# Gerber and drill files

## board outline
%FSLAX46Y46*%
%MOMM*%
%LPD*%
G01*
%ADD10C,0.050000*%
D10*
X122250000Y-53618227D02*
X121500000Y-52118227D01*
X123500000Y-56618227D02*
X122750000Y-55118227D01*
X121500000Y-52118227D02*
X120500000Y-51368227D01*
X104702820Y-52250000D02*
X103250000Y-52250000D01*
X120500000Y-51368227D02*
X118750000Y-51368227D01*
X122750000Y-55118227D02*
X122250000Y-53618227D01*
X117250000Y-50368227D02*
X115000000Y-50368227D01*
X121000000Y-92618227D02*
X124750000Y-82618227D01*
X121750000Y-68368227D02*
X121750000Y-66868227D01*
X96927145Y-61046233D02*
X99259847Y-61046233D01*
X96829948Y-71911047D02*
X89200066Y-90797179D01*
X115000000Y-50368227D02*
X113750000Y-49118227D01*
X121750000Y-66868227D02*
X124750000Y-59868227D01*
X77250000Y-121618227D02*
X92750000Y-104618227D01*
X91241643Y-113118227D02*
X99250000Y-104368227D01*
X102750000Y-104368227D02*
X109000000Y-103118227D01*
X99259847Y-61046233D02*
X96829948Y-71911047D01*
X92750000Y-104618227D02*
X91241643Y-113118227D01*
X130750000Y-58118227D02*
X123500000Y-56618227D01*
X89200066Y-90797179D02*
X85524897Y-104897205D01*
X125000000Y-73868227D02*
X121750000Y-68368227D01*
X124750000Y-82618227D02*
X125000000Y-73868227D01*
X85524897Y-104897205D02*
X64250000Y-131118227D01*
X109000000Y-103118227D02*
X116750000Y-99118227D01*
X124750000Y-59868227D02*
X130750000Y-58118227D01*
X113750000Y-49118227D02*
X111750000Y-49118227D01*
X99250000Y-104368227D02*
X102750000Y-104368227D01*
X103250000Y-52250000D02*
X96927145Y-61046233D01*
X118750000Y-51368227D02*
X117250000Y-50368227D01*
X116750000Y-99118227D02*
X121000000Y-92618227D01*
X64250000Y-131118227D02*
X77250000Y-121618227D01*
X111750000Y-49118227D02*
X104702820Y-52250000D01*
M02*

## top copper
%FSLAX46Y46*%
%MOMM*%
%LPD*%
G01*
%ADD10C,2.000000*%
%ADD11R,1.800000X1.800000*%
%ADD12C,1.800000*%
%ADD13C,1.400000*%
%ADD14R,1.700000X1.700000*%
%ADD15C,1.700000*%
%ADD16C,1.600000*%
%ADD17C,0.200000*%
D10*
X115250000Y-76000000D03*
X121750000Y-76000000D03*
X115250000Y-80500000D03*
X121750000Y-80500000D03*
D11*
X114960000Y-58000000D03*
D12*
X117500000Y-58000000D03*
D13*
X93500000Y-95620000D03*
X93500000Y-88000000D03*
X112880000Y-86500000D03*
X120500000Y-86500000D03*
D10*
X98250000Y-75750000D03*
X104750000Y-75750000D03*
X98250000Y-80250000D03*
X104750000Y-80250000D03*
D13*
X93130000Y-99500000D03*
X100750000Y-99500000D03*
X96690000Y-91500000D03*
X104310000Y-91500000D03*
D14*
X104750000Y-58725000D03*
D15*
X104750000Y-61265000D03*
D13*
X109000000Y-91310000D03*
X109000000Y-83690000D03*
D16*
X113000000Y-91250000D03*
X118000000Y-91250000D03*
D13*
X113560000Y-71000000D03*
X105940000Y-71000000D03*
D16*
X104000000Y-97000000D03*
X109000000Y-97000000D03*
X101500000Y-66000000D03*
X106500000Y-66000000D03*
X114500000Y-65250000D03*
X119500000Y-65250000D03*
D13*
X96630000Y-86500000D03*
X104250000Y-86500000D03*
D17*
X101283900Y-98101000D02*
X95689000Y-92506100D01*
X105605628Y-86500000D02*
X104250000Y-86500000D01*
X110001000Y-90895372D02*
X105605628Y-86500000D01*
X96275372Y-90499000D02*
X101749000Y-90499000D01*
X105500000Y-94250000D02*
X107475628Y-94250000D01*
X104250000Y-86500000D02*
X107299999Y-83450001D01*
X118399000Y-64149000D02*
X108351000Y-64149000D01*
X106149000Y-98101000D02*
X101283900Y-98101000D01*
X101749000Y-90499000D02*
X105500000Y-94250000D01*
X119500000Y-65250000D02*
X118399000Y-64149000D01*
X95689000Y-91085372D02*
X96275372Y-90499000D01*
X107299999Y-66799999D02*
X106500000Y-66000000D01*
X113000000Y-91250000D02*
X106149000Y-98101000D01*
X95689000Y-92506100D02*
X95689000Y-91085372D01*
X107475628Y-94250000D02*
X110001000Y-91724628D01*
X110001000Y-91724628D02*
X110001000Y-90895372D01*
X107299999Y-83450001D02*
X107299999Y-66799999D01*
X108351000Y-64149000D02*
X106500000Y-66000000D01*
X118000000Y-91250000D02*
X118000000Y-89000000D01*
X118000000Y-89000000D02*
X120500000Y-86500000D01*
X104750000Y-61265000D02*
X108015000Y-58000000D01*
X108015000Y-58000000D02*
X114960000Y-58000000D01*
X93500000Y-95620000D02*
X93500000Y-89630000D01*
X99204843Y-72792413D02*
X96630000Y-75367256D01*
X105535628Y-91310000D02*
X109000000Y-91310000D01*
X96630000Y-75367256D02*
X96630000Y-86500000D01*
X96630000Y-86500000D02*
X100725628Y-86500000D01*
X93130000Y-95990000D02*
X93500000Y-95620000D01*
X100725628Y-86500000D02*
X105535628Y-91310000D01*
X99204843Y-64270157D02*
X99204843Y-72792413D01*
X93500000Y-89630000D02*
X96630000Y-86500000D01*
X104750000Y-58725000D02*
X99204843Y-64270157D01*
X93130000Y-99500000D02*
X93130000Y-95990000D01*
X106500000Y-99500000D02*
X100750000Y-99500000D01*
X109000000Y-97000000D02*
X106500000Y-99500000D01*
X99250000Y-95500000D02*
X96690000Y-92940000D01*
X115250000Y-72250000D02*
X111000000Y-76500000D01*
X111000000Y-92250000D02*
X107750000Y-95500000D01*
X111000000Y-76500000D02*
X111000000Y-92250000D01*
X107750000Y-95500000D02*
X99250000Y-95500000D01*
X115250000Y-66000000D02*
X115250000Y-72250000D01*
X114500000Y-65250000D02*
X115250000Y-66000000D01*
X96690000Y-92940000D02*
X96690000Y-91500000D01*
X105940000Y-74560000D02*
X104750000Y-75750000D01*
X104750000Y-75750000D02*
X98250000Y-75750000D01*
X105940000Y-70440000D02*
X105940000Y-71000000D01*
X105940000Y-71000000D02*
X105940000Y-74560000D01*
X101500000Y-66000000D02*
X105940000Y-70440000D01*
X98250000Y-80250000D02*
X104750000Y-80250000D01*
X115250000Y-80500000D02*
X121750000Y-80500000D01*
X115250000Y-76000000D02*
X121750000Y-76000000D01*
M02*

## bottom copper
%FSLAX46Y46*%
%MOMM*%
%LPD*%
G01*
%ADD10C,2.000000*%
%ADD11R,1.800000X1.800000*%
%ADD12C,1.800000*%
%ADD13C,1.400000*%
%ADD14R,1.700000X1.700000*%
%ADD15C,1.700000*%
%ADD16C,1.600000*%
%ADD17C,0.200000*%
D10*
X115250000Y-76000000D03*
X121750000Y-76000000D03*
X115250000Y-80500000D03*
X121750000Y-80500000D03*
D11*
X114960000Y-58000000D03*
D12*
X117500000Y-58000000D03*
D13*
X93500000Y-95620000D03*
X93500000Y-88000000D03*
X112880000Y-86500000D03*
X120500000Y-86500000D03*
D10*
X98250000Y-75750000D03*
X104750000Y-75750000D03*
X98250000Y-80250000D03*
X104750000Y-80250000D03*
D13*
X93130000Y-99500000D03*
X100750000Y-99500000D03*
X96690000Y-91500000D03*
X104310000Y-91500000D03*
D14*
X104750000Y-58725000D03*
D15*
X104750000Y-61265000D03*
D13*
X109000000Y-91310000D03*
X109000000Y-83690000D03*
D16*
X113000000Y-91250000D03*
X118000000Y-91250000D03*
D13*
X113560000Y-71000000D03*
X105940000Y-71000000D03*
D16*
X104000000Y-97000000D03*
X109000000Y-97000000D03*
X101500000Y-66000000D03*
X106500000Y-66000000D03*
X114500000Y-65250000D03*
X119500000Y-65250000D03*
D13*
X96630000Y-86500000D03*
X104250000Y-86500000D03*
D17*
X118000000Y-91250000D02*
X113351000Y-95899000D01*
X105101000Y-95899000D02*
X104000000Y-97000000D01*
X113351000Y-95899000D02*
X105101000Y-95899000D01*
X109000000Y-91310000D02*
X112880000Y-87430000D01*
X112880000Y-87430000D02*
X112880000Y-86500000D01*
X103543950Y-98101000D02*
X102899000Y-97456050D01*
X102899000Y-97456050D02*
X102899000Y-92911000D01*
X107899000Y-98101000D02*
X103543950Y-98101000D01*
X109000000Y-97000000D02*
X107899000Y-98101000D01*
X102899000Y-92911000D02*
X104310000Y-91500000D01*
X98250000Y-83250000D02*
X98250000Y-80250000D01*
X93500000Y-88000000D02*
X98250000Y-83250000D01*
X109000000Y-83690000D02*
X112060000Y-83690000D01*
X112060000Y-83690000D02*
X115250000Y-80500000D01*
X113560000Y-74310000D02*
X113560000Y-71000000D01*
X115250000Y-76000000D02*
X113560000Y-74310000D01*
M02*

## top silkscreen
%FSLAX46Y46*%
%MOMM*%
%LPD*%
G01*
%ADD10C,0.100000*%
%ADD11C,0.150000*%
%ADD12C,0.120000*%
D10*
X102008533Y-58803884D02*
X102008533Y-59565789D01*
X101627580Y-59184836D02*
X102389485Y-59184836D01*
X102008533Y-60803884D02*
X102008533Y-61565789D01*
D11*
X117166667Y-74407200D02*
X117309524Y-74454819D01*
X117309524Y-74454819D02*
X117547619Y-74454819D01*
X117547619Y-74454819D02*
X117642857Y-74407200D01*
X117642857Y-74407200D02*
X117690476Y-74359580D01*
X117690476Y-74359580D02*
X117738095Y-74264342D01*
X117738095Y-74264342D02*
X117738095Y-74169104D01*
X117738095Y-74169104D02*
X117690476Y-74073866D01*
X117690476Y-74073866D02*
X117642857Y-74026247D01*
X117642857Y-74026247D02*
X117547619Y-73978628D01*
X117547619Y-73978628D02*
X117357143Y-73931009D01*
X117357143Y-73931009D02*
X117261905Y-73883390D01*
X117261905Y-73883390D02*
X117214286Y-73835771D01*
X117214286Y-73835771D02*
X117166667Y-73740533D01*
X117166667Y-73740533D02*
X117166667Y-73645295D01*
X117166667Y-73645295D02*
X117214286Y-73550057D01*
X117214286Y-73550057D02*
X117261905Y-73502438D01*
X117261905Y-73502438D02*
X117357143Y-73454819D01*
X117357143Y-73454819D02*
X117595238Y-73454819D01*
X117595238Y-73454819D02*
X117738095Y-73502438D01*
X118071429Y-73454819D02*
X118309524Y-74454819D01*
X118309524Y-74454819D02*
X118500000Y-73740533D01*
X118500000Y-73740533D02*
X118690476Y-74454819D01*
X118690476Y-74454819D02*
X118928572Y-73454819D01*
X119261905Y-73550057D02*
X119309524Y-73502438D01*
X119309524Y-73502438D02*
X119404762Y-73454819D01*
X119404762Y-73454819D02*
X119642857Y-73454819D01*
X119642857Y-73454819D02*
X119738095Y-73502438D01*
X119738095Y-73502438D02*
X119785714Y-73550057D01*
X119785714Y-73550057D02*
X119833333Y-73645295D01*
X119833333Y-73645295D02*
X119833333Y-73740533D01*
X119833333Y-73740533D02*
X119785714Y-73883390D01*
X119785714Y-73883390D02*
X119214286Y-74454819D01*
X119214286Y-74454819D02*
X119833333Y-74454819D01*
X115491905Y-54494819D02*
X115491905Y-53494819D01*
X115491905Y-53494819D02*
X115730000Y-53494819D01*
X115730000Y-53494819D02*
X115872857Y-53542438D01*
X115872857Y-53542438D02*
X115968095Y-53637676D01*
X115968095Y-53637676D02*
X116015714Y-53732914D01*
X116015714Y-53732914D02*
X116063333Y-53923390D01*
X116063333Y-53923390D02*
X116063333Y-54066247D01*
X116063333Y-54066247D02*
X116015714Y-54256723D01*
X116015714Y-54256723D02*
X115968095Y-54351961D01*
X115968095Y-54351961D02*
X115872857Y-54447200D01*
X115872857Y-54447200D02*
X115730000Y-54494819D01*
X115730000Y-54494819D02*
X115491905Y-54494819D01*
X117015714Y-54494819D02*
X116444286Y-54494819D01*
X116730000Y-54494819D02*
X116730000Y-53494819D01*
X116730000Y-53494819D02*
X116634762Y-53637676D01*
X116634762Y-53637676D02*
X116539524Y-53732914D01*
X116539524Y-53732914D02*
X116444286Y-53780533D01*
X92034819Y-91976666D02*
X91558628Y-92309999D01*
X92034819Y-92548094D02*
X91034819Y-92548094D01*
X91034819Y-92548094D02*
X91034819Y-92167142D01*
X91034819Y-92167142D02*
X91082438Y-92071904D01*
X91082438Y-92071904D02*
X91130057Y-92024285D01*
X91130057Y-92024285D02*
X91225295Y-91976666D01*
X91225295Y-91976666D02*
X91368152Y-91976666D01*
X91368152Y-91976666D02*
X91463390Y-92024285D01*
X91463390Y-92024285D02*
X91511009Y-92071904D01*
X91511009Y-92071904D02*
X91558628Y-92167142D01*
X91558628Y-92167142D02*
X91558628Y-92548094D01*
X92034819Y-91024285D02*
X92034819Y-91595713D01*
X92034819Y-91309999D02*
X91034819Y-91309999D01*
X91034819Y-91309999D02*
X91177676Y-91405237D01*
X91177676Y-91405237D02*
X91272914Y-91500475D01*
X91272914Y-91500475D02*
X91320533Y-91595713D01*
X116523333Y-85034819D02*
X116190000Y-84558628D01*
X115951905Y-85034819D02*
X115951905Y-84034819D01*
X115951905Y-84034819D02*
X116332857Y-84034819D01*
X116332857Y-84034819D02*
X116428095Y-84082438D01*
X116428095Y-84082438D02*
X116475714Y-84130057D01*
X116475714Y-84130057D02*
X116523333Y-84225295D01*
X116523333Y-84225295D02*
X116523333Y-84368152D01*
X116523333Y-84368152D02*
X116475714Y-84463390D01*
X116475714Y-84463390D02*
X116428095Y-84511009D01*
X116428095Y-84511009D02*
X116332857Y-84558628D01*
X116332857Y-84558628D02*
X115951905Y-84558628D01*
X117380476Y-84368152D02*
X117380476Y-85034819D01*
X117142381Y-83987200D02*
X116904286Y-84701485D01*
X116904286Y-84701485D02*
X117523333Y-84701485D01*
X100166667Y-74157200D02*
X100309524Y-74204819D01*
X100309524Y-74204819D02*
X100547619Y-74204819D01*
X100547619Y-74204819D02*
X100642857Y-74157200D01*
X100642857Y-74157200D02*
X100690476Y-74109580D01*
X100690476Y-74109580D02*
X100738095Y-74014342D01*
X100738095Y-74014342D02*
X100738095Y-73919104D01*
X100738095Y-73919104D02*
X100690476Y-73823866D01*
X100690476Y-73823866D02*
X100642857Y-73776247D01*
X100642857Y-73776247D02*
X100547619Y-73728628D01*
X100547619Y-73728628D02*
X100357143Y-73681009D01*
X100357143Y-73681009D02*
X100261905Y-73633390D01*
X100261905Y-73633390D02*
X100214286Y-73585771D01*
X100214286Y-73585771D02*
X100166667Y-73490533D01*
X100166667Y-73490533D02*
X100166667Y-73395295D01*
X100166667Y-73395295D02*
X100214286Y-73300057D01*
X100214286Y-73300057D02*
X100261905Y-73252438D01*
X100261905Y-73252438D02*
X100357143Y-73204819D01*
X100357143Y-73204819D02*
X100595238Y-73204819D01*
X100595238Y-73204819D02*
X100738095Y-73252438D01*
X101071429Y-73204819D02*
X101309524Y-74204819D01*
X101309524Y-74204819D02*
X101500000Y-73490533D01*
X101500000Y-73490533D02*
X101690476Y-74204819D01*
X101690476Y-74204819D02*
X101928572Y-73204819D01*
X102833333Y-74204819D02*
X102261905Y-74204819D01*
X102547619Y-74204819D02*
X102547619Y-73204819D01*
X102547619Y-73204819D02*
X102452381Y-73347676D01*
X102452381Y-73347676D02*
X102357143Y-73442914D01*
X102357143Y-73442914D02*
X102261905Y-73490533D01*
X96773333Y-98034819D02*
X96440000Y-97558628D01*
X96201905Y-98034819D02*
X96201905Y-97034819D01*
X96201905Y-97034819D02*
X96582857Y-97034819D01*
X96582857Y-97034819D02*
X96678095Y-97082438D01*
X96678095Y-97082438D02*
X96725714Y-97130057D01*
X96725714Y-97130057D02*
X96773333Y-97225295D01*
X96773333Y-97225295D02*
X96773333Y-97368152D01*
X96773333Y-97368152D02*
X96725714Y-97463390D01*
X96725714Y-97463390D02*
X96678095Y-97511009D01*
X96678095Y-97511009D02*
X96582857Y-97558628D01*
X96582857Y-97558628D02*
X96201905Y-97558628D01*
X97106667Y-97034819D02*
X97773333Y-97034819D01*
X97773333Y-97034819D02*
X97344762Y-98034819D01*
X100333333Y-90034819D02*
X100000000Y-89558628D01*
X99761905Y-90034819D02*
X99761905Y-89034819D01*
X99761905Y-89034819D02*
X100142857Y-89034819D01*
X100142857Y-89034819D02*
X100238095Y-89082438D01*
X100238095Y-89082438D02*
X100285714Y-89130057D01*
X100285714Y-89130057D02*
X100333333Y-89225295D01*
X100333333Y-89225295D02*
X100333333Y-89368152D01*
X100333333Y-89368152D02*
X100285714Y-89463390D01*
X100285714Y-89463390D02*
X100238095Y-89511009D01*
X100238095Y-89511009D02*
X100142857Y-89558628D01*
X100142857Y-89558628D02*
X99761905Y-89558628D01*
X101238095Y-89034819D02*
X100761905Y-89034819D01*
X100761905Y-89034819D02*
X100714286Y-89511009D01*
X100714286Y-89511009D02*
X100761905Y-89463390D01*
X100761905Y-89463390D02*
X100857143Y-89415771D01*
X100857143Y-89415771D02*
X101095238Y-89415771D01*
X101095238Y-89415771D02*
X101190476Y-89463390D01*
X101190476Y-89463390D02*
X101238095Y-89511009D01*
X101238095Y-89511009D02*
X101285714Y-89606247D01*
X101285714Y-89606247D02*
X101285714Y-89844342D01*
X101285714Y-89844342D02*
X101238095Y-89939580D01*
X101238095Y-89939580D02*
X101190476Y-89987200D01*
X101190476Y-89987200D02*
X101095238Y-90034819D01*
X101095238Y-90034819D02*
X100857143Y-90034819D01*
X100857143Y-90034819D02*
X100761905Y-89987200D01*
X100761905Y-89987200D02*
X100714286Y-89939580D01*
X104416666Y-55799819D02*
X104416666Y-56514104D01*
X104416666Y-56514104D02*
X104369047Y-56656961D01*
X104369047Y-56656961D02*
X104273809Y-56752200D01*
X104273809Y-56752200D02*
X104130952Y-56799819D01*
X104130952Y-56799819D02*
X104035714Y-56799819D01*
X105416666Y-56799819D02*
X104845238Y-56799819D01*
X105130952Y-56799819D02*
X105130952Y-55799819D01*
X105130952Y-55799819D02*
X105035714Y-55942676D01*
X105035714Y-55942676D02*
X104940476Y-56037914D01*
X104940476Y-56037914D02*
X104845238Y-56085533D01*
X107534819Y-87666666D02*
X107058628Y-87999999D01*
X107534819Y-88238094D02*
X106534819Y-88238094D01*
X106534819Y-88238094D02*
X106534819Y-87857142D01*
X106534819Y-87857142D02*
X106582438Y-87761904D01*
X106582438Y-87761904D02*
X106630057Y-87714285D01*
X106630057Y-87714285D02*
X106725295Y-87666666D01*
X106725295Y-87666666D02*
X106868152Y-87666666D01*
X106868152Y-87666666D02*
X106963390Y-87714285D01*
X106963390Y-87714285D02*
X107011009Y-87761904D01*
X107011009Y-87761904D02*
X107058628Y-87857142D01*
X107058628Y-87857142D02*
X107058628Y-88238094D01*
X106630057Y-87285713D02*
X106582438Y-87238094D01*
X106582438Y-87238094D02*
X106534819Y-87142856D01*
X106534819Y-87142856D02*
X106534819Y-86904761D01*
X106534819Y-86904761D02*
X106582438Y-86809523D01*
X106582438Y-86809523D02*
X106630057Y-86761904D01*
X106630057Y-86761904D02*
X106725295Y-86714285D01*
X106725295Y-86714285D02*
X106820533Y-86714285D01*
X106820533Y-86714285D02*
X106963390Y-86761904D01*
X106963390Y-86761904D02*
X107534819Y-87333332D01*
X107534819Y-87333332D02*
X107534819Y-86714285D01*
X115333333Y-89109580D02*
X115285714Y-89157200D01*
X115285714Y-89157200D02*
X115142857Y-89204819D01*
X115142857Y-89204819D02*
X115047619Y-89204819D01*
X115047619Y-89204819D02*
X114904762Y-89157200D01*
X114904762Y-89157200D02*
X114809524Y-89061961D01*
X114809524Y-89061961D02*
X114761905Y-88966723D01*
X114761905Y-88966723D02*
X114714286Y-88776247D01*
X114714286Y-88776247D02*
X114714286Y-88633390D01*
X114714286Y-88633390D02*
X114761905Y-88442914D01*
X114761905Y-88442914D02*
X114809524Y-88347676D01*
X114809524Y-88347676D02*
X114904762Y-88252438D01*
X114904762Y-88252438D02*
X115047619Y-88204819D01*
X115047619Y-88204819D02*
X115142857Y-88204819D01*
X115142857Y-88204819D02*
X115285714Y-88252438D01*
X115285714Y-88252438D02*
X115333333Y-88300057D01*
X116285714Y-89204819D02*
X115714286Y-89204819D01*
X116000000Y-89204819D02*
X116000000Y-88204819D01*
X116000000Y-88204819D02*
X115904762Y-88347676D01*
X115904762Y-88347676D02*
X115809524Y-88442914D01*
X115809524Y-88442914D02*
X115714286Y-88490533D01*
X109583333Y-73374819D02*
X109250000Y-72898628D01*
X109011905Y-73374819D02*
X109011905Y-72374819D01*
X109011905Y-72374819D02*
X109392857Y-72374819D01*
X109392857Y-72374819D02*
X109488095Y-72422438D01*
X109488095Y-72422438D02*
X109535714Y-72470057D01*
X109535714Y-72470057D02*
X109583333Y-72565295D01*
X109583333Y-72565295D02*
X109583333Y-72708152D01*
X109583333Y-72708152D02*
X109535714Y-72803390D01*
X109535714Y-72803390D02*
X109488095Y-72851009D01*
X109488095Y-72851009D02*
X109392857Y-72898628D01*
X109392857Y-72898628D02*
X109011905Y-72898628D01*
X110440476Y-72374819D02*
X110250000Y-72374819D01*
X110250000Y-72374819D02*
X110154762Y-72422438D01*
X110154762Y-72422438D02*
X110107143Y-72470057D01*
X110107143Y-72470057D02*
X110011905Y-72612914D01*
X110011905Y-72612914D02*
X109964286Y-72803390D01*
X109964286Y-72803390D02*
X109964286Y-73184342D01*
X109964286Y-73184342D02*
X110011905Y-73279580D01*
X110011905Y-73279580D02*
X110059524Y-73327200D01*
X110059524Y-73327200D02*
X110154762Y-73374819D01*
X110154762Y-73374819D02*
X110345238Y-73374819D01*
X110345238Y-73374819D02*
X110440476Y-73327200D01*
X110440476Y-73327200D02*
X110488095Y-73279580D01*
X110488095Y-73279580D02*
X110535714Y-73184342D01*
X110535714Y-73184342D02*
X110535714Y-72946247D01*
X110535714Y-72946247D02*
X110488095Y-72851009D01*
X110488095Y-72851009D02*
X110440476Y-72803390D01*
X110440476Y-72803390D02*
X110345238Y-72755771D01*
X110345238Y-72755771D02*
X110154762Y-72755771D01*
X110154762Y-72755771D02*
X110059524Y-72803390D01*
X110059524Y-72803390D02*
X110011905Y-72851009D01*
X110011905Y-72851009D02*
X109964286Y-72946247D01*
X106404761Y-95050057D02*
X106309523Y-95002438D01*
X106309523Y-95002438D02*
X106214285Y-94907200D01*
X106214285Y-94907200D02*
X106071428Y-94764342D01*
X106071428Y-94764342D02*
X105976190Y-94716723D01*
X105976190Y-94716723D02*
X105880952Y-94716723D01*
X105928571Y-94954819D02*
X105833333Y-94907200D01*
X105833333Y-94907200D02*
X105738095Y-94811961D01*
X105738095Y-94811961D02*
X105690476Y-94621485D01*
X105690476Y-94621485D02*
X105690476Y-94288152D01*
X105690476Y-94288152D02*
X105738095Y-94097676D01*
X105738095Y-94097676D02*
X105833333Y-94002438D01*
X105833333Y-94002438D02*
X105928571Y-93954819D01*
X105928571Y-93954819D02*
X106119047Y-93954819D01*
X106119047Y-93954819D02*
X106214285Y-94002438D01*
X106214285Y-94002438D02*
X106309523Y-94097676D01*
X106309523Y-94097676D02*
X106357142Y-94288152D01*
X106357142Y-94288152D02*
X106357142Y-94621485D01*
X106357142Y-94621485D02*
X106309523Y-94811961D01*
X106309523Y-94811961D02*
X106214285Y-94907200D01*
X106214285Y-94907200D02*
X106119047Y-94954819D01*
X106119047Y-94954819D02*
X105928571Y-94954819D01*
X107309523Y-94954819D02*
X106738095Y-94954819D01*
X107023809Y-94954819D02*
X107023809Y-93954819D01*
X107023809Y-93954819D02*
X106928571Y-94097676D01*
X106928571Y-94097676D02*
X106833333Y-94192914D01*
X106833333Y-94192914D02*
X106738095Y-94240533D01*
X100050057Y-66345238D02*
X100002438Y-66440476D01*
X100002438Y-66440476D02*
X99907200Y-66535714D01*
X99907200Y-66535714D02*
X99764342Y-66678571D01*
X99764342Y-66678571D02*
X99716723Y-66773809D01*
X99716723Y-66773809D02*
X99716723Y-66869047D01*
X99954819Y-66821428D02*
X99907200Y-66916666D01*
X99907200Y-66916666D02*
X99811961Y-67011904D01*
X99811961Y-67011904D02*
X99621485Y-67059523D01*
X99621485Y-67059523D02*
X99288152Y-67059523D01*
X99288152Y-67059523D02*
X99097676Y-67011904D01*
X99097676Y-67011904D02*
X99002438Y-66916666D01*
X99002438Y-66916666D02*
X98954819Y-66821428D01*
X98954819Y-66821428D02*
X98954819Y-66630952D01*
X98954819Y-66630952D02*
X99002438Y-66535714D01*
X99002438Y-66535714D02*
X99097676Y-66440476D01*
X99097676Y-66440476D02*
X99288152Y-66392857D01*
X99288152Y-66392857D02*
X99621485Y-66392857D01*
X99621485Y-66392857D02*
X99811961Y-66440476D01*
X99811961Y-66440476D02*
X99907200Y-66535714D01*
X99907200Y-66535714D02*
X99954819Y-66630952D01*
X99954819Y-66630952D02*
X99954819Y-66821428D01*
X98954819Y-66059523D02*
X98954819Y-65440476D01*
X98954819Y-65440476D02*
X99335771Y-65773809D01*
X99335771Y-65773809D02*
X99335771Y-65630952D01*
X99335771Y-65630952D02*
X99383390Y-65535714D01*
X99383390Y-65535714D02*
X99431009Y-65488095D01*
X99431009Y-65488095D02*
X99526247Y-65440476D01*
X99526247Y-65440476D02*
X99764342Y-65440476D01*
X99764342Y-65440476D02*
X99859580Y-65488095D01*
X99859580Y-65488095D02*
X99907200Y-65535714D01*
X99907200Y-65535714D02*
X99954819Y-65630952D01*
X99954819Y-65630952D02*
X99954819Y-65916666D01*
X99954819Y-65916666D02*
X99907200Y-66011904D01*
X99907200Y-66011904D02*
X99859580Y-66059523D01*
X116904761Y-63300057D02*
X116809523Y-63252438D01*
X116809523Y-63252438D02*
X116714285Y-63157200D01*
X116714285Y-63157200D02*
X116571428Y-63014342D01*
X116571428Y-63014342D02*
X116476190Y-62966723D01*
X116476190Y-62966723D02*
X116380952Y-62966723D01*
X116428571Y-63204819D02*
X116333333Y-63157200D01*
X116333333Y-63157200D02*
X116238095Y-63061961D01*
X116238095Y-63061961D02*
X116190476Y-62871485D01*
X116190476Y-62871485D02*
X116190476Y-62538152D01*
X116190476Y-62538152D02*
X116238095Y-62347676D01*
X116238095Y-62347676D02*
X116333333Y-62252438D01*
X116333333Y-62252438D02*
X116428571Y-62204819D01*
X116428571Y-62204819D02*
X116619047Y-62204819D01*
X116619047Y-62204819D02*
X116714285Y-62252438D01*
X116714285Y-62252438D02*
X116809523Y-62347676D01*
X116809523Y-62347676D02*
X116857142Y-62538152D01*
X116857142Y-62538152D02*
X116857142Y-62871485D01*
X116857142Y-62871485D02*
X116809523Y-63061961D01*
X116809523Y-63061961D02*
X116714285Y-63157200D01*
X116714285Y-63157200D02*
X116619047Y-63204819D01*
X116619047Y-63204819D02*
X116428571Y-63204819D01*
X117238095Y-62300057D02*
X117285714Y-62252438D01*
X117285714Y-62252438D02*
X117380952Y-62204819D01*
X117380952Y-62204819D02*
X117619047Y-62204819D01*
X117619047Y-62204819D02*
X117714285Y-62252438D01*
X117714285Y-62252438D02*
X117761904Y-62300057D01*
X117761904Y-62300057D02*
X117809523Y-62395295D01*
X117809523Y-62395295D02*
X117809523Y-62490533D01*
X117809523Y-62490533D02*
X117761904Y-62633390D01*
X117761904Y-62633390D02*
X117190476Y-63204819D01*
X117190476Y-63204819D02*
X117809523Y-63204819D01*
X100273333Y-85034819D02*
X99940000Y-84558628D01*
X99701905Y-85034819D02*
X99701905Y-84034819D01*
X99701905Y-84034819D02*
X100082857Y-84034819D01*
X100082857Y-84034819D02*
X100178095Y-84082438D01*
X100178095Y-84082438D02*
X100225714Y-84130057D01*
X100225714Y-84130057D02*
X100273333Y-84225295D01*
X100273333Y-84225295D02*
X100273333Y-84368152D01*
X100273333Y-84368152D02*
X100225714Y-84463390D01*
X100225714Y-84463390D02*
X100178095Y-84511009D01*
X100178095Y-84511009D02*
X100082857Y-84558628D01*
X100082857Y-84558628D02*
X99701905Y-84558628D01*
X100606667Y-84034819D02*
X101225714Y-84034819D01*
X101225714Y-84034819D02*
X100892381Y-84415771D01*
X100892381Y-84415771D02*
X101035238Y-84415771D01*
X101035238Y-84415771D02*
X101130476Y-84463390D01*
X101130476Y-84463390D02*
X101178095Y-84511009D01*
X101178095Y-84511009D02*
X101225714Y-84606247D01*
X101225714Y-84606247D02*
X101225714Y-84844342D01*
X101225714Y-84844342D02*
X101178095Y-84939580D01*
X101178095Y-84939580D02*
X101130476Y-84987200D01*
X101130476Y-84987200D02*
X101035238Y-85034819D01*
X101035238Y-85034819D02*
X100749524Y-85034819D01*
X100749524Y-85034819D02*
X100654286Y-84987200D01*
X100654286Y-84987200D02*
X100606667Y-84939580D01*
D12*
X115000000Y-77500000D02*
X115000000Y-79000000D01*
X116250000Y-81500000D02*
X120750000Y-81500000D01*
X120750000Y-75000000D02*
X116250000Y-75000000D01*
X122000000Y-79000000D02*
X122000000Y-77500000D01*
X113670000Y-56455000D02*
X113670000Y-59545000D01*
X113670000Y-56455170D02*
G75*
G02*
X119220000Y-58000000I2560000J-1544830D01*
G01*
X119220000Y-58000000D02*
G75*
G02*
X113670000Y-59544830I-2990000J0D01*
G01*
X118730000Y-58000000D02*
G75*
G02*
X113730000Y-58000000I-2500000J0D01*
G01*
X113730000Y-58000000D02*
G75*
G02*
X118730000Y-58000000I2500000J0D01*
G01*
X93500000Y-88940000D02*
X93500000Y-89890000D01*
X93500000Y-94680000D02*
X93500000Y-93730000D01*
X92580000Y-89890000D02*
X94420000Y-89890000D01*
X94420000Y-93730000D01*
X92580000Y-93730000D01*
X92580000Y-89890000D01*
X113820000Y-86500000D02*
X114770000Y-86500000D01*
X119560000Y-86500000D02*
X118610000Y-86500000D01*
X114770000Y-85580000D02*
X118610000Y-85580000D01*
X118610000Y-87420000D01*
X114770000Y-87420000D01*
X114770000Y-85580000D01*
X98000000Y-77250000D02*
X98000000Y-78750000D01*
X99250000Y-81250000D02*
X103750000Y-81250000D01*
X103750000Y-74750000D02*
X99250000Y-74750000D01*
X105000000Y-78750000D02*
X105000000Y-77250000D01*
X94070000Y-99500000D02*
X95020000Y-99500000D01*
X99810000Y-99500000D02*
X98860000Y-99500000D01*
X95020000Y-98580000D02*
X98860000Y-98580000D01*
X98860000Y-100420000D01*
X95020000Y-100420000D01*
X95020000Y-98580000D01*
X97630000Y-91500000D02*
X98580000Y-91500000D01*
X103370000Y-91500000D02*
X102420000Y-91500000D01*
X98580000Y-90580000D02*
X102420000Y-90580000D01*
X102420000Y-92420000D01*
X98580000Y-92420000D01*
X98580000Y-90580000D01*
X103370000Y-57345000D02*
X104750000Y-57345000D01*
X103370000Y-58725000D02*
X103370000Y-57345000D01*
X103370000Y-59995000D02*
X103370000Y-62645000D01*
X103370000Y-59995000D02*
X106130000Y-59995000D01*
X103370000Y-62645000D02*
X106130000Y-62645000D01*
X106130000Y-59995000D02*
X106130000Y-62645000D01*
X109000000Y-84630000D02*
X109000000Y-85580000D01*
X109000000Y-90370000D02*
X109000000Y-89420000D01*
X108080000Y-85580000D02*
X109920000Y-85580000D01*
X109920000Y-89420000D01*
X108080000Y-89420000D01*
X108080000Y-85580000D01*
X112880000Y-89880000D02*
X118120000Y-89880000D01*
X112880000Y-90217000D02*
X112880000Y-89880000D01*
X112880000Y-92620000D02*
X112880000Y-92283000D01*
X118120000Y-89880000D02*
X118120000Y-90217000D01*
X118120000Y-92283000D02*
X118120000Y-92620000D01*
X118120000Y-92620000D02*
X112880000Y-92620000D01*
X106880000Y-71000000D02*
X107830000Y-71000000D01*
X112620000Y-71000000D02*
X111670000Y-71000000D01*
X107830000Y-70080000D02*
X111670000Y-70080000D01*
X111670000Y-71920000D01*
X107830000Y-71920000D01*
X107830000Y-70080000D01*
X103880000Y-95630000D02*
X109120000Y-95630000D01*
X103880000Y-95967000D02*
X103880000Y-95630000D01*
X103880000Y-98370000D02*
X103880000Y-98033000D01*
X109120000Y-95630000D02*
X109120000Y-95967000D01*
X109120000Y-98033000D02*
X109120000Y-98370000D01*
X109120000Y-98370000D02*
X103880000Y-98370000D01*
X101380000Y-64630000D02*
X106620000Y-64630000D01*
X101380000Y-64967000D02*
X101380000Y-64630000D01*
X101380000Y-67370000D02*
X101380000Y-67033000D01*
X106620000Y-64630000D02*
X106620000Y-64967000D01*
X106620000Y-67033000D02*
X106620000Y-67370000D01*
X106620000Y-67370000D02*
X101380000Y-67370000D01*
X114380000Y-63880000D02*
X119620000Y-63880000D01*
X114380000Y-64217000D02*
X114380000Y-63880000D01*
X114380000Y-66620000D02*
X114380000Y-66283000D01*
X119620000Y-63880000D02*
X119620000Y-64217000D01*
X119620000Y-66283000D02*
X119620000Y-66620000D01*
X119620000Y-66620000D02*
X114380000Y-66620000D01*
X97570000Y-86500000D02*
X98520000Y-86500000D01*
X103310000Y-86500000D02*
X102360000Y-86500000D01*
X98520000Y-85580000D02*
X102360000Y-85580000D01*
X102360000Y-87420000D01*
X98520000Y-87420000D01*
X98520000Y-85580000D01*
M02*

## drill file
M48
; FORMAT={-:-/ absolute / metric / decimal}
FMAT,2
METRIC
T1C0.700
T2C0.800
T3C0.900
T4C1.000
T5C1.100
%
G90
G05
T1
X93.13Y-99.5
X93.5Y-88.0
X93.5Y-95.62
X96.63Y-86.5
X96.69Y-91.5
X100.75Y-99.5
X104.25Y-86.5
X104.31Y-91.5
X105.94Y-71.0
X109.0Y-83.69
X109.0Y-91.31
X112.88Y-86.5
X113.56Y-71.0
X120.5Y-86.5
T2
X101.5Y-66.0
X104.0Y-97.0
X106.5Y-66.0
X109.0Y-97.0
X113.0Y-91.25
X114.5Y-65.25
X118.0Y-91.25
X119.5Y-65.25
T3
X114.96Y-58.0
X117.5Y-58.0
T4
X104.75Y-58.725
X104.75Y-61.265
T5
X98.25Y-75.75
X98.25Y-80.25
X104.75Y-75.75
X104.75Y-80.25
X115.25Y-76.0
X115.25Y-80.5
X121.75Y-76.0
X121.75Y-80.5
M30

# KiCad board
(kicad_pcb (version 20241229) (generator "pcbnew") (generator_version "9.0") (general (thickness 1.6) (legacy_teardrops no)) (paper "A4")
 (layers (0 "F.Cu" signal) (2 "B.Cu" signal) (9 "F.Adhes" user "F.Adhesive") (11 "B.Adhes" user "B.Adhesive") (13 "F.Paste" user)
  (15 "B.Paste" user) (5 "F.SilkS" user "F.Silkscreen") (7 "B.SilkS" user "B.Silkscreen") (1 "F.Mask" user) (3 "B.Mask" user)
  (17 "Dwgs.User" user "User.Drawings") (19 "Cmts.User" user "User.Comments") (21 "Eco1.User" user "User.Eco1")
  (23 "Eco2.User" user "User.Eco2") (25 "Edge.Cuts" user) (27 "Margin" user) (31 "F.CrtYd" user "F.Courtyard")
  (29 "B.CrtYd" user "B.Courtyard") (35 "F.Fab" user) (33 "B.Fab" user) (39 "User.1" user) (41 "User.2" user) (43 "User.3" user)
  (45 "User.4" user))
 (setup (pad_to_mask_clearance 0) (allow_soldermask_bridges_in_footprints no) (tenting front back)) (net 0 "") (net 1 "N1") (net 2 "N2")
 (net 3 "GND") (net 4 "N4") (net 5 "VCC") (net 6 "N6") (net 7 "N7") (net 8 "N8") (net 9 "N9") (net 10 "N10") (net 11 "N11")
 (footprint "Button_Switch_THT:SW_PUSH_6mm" (layer "F.Cu") (at 115.25 76)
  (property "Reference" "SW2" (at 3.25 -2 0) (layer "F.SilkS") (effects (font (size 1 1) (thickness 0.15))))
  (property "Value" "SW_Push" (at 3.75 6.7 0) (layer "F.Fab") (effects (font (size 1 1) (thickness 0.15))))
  (fp_line (start -0.25 1.5) (end -0.25 3) (stroke (width 0.12) (type solid)) (layer "F.SilkS"))
  (fp_line (start 1 5.5) (end 5.5 5.5) (stroke (width 0.12) (type solid)) (layer "F.SilkS"))
  (fp_line (start 5.5 -1) (end 1 -1) (stroke (width 0.12) (type solid)) (layer "F.SilkS"))
  (fp_line (start 6.75 3) (end 6.75 1.5) (stroke (width 0.12) (type solid)) (layer "F.SilkS"))
  (pad "1" thru_hole circle (at 0 0 90) (size 2 2) (drill 1.1) (layers "*.Cu" "*.Mask") (remove_unused_layers no) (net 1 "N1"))
  (pad "1" thru_hole circle (at 6.5 0 90) (size 2 2) (drill 1.1) (layers "*.Cu" "*.Mask") (remove_unused_layers no) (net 1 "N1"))
  (pad "2" thru_hole circle (at 0 4.5 90) (size 2 2) (drill 1.1) (layers "*.Cu" "*.Mask") (remove_unused_layers no) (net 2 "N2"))
  (pad "2" thru_hole circle (at 6.5 4.5 90) (size 2 2) (drill 1.1) (layers "*.Cu" "*.Mask") (remove_unused_layers no) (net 2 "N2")))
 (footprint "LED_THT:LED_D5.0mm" (layer "F.Cu") (at 114.96 58)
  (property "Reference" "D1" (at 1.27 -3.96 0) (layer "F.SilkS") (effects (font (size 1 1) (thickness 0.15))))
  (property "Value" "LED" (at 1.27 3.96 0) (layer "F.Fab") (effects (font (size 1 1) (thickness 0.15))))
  (fp_line (start -1.29 -1.545) (end -1.29 1.545) (stroke (width 0.12) (type solid)) (layer "F.SilkS"))
  (fp_arc (start -1.29 -1.54483) (mid 2.071779 -2.880495) (end 4.26 0) (stroke (width 0.12) (type solid)) (layer "F.SilkS"))
  (fp_arc (start 4.26 0) (mid 2.071779 2.880495) (end -1.29 1.54483) (stroke (width 0.12) (type solid)) (layer "F.SilkS"))
  (fp_circle (center 1.27 0) (end 3.77 0) (stroke (width 0.12) (type solid)) (fill no) (layer "F.SilkS"))
  (pad "1" thru_hole rect (at 0 0) (size 1.8 1.8) (drill 0.9) (layers "*.Cu" "*.Mask") (remove_unused_layers no) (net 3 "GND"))
  (pad "2" thru_hole circle (at 2.54 0) (size 1.8 1.8) (drill 0.9) (layers "*.Cu" "*.Mask") (remove_unused_layers no) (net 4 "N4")))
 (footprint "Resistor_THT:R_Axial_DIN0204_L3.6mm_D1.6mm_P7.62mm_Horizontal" (layer "F.Cu") (at 93.5 95.62 90)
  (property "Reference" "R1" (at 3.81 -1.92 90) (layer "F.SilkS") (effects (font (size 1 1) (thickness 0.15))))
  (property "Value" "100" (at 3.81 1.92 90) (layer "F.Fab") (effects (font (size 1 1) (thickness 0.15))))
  (fp_line (start 6.68 0) (end 5.73 0) (stroke (width 0.12) (type solid)) (layer "F.SilkS"))
  (fp_line (start 0.94 0) (end 1.89 0) (stroke (width 0.12) (type solid)) (layer "F.SilkS"))
  (fp_rect (start 1.89 -0.92) (end 5.73 0.92) (stroke (width 0.12) (type solid)) (fill no) (layer "F.SilkS"))
  (pad "1" thru_hole circle (at 0 0 90) (size 1.4 1.4) (drill 0.7) (layers "*.Cu" "*.Mask") (remove_unused_layers no) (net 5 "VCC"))
  (pad "2" thru_hole circle (at 7.62 0 90) (size 1.4 1.4) (drill 0.7) (layers "*.Cu" "*.Mask") (remove_unused_layers no) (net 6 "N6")))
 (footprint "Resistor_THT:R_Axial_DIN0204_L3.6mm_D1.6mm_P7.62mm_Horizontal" (layer "F.Cu") (at 112.88 86.5)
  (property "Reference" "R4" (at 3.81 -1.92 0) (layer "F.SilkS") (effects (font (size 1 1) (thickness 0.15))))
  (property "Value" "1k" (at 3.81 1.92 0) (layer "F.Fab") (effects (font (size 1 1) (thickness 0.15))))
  (fp_line (start 0.94 0) (end 1.89 0) (stroke (width 0.12) (type solid)) (layer "F.SilkS"))
  (fp_line (start 6.68 0) (end 5.73 0) (stroke (width 0.12) (type solid)) (layer "F.SilkS"))
  (fp_rect (start 1.89 -0.92) (end 5.73 0.92) (stroke (width 0.12) (type solid)) (fill no) (layer "F.SilkS"))
  (pad "1" thru_hole circle (at 0 0) (size 1.4 1.4) (drill 0.7) (layers "*.Cu" "*.Mask") (remove_unused_layers no) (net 5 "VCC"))
  (pad "2" thru_hole circle (at 7.62 0) (size 1.4 1.4) (drill 0.7) (layers "*.Cu" "*.Mask") (remove_unused_layers no) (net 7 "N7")))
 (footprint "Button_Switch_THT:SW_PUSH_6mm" (layer "F.Cu") (at 98.25 75.75)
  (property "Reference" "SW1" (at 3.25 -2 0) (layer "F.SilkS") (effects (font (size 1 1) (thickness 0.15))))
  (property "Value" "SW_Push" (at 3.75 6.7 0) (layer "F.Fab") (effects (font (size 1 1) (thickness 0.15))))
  (fp_line (start -0.25 1.5) (end -0.25 3) (stroke (width 0.12) (type solid)) (layer "F.SilkS"))
  (fp_line (start 1 5.5) (end 5.5 5.5) (stroke (width 0.12) (type solid)) (layer "F.SilkS"))
  (fp_line (start 5.5 -1) (end 1 -1) (stroke (width 0.12) (type solid)) (layer "F.SilkS"))
  (fp_line (start 6.75 3) (end 6.75 1.5) (stroke (width 0.12) (type solid)) (layer "F.SilkS"))
  (pad "1" thru_hole circle (at 0 0 90) (size 2 2) (drill 1.1) (layers "*.Cu" "*.Mask") (remove_unused_layers no) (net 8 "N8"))
  (pad "1" thru_hole circle (at 6.5 0 90) (size 2 2) (drill 1.1) (layers "*.Cu" "*.Mask") (remove_unused_layers no) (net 8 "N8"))
  (pad "2" thru_hole circle (at 0 4.5 90) (size 2 2) (drill 1.1) (layers "*.Cu" "*.Mask") (remove_unused_layers no) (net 6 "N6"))
  (pad "2" thru_hole circle (at 6.5 4.5 90) (size 2 2) (drill 1.1) (layers "*.Cu" "*.Mask") (remove_unused_layers no) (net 6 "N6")))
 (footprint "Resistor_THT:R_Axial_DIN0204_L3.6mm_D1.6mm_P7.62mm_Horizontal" (layer "F.Cu") (at 93.13 99.5)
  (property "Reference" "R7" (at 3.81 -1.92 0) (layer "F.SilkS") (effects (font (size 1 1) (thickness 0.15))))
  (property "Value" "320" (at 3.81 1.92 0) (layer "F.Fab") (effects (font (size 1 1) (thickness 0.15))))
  (fp_line (start 0.94 0) (end 1.89 0) (stroke (width 0.12) (type solid)) (layer "F.SilkS"))
  (fp_line (start 6.68 0) (end 5.73 0) (stroke (width 0.12) (type solid)) (layer "F.SilkS"))
  (fp_rect (start 1.89 -0.92) (end 5.73 0.92) (stroke (width 0.12) (type solid)) (fill no) (layer "F.SilkS"))
  (pad "1" thru_hole circle (at 0 0) (size 1.4 1.4) (drill 0.7) (layers "*.Cu" "*.Mask") (remove_unused_layers no) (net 5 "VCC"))
  (pad "2" thru_hole circle (at 7.62 0) (size 1.4 1.4) (drill 0.7) (layers "*.Cu" "*.Mask") (remove_unused_layers no) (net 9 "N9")))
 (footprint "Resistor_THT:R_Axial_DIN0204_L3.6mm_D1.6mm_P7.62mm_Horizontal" (layer "F.Cu") (at 96.69 91.5)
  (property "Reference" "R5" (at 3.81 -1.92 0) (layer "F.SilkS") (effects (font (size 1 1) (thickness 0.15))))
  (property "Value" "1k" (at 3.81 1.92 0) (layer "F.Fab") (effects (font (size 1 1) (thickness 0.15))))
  (fp_line (start 0.94 0) (end 1.89 0) (stroke (width 0.12) (type solid)) (layer "F.SilkS"))
  (fp_line (start 6.68 0) (end 5.73 0) (stroke (width 0.12) (type solid)) (layer "F.SilkS"))
  (fp_rect (start 1.89 -0.92) (end 5.73 0.92) (stroke (width 0.12) (type solid)) (fill no) (layer "F.SilkS"))
  (pad "1" thru_hole circle (at 0 0) (size 1.4 1.4) (drill 0.7) (layers "*.Cu" "*.Mask") (remove_unused_layers no) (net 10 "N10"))
  (pad "2" thru_hole circle (at 7.62 0) (size 1.4 1.4) (drill 0.7) (layers "*.Cu" "*.Mask") (remove_unused_layers no) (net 9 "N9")))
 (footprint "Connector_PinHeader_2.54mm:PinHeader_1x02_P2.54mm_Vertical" (layer "F.Cu") (at 104.75 58.725)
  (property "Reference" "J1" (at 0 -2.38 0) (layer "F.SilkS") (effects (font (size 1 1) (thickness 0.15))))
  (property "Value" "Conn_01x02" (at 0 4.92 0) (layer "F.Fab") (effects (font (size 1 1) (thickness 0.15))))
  (fp_line (start -1.38 -1.38) (end 0 -1.38) (stroke (width 0.12) (type solid)) (layer "F.SilkS"))
  (fp_line (start -1.38 0) (end -1.38 -1.38) (stroke (width 0.12) (type solid)) (layer "F.SilkS"))
  (fp_line (start -1.38 1.27) (end -1.38 3.92) (stroke (width 0.12) (type solid)) (layer "F.SilkS"))
  (fp_line (start -1.38 1.27) (end 1.38 1.27) (stroke (width 0.12) (type solid)) (layer "F.SilkS"))
  (fp_line (start -1.38 3.92) (end 1.38 3.92) (stroke (width 0.12) (type solid)) (layer "F.SilkS"))
  (fp_line (start 1.38 1.27) (end 1.38 3.92) (stroke (width 0.12) (type solid)) (layer "F.SilkS"))
  (pad "1" thru_hole rect (at 0 0) (size 1.7 1.7) (drill 1) (layers "*.Cu" "*.Mask") (remove_unused_layers no) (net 5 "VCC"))
  (pad "2" thru_hole circle (at 0 2.54) (size 1.7 1.7) (drill 1) (layers "*.Cu" "*.Mask") (remove_unused_layers no) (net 3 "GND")))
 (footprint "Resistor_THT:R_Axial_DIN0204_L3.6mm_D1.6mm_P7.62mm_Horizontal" (layer "F.Cu") (at 109 91.31 90)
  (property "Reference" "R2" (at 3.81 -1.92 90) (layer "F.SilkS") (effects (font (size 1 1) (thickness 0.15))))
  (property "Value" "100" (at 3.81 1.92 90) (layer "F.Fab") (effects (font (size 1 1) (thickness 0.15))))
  (fp_line (start 6.68 0) (end 5.73 0) (stroke (width 0.12) (type solid)) (layer "F.SilkS"))
  (fp_line (start 0.94 0) (end 1.89 0) (stroke (width 0.12) (type solid)) (layer "F.SilkS"))
  (fp_rect (start 1.89 -0.92) (end 5.73 0.92) (stroke (width 0.12) (type solid)) (fill no) (layer "F.SilkS"))
  (pad "1" thru_hole circle (at 0 0 90) (size 1.4 1.4) (drill 0.7) (layers "*.Cu" "*.Mask") (remove_unused_layers no) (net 5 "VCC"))
  (pad "2" thru_hole circle (at 7.62 0 90) (size 1.4 1.4) (drill 0.7) (layers "*.Cu" "*.Mask") (remove_unused_layers no) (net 2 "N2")))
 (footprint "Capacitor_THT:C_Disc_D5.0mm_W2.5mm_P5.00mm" (layer "F.Cu") (at 113 91.25)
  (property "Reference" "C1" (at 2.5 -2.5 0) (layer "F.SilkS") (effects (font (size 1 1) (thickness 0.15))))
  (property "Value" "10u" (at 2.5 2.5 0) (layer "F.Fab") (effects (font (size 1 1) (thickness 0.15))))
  (fp_line (start -0.12 -1.37) (end 5.12 -1.37) (stroke (width 0.12) (type solid)) (layer "F.SilkS"))
  (fp_line (start -0.12 -1.033) (end -0.12 -1.37) (stroke (width 0.12) (type solid)) (layer "F.SilkS"))
  (fp_line (start -0.12 1.37) (end -0.12 1.033) (stroke (width 0.12) (type solid)) (layer "F.SilkS"))
  (fp_line (start 5.12 -1.37) (end 5.12 -1.033) (stroke (width 0.12) (type solid)) (layer "F.SilkS"))
  (fp_line (start 5.12 1.033) (end 5.12 1.37) (stroke (width 0.12) (type solid)) (layer "F.SilkS"))
  (fp_line (start 5.12 1.37) (end -0.12 1.37) (stroke (width 0.12) (type solid)) (layer "F.SilkS"))
  (pad "1" thru_hole circle (at 0 0) (size 1.6 1.6) (drill 0.8) (layers "*.Cu" "*.Mask") (remove_unused_layers no) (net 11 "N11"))
  (pad "2" thru_hole circle (at 5 0) (size 1.6 1.6) (drill 0.8) (layers "*.Cu" "*.Mask") (remove_unused_layers no) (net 7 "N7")))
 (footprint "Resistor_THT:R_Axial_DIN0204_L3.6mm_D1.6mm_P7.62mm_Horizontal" (layer "F.Cu") (at 113.56 71 180)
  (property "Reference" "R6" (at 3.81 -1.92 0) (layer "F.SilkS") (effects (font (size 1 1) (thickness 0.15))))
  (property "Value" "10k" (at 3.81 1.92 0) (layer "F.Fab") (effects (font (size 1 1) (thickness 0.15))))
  (fp_line (start 6.68 0) (end 5.73 0) (stroke (width 0.12) (type solid)) (layer "F.SilkS"))
  (fp_line (start 0.94 0) (end 1.89 0) (stroke (width 0.12) (type solid)) (layer "F.SilkS"))
  (fp_rect (start 1.89 -0.92) (end 5.73 0.92) (stroke (width 0.12) (type solid)) (fill no) (layer "F.SilkS"))
  (pad "1" thru_hole circle (at 0 0 180) (size 1.4 1.4) (drill 0.7) (layers "*.Cu" "*.Mask") (remove_unused_layers no) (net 1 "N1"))
  (pad "2" thru_hole circle (at 7.62 0 180) (size 1.4 1.4) (drill 0.7) (layers "*.Cu" "*.Mask") (remove_unused_layers no) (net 8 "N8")))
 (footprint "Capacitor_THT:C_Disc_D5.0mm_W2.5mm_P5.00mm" (layer "F.Cu") (at 104 97)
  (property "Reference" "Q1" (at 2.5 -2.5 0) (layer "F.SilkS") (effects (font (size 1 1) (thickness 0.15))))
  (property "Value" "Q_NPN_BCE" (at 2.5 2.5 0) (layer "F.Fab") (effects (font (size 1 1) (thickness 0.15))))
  (fp_line (start -0.12 -1.37) (end 5.12 -1.37) (stroke (width 0.12) (type solid)) (layer "F.SilkS"))
  (fp_line (start -0.12 -1.033) (end -0.12 -1.37) (stroke (width 0.12) (type solid)) (layer "F.SilkS"))
  (fp_line (start -0.12 1.37) (end -0.12 1.033) (stroke (width 0.12) (type solid)) (layer "F.SilkS"))
  (fp_line (start 5.12 -1.37) (end 5.12 -1.033) (stroke (width 0.12) (type solid)) (layer "F.SilkS"))
  (fp_line (start 5.12 1.033) (end 5.12 1.37) (stroke (width 0.12) (type solid)) (layer "F.SilkS"))
  (fp_line (start 5.12 1.37) (end -0.12 1.37) (stroke (width 0.12) (type solid)) (layer "F.SilkS"))
  (pad "1" thru_hole circle (at 0 0) (size 1.6 1.6) (drill 0.8) (layers "*.Cu" "*.Mask") (remove_unused_layers no) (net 7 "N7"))
  (pad "2" thru_hole circle (at 5 0) (size 1.6 1.6) (drill 0.8) (layers "*.Cu" "*.Mask") (remove_unused_layers no) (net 9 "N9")))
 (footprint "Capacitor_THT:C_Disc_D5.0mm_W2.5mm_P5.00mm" (layer "F.Cu") (at 101.5 66)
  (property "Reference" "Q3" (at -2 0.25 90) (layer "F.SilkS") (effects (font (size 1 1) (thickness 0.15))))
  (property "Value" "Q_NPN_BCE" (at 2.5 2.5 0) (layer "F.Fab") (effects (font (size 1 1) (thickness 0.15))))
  (fp_line (start -0.12 -1.37) (end 5.12 -1.37) (stroke (width 0.12) (type solid)) (layer "F.SilkS"))
  (fp_line (start -0.12 -1.033) (end -0.12 -1.37) (stroke (width 0.12) (type solid)) (layer "F.SilkS"))
  (fp_line (start -0.12 1.37) (end -0.12 1.033) (stroke (width 0.12) (type solid)) (layer "F.SilkS"))
  (fp_line (start 5.12 -1.37) (end 5.12 -1.033) (stroke (width 0.12) (type solid)) (layer "F.SilkS"))
  (fp_line (start 5.12 1.033) (end 5.12 1.37) (stroke (width 0.12) (type solid)) (layer "F.SilkS"))
  (fp_line (start 5.12 1.37) (end -0.12 1.37) (stroke (width 0.12) (type solid)) (layer "F.SilkS"))
  (pad "1" thru_hole circle (at 0 0) (size 1.6 1.6) (drill 0.8) (layers "*.Cu" "*.Mask") (remove_unused_layers no) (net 8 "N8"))
  (pad "2" thru_hole circle (at 5 0) (size 1.6 1.6) (drill 0.8) (layers "*.Cu" "*.Mask") (remove_unused_layers no) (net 11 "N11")))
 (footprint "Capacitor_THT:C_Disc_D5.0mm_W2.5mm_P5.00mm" (layer "F.Cu") (at 114.5 65.25)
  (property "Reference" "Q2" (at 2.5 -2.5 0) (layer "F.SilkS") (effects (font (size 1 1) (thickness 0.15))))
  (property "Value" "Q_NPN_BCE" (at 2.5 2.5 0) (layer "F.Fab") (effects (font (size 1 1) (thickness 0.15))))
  (fp_line (start -0.12 -1.37) (end 5.12 -1.37) (stroke (width 0.12) (type solid)) (layer "F.SilkS"))
  (fp_line (start -0.12 -1.033) (end -0.12 -1.37) (stroke (width 0.12) (type solid)) (layer "F.SilkS"))
  (fp_line (start -0.12 1.37) (end -0.12 1.033) (stroke (width 0.12) (type solid)) (layer "F.SilkS"))
  (fp_line (start 5.12 -1.37) (end 5.12 -1.033) (stroke (width 0.12) (type solid)) (layer "F.SilkS"))
  (fp_line (start 5.12 1.033) (end 5.12 1.37) (stroke (width 0.12) (type solid)) (layer "F.SilkS"))
  (fp_line (start 5.12 1.37) (end -0.12 1.37) (stroke (width 0.12) (type solid)) (layer "F.SilkS"))
  (pad "1" thru_hole circle (at 0 0) (size 1.6 1.6) (drill 0.8) (layers "*.Cu" "*.Mask") (remove_unused_layers no) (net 10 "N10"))
  (pad "2" thru_hole circle (at 5 0) (size 1.6 1.6) (drill 0.8) (layers "*.Cu" "*.Mask") (remove_unused_layers no) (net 11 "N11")))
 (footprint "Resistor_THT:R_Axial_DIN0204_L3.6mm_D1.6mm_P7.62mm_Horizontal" (layer "F.Cu") (at 96.63 86.5)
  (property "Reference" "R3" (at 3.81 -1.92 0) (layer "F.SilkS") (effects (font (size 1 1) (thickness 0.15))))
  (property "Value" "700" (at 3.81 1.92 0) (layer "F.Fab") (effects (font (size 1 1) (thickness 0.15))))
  (fp_line (start 0.94 0) (end 1.89 0) (stroke (width 0.12) (type solid)) (layer "F.SilkS"))
  (fp_line (start 6.68 0) (end 5.73 0) (stroke (width 0.12) (type solid)) (layer "F.SilkS"))
  (fp_rect (start 1.89 -0.92) (end 5.73 0.92) (stroke (width 0.12) (type solid)) (fill no) (layer "F.SilkS"))
  (pad "1" thru_hole circle (at 0 0) (size 1.4 1.4) (drill 0.7) (layers "*.Cu" "*.Mask") (remove_unused_layers no) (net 5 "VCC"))
  (pad "2" thru_hole circle (at 7.62 0) (size 1.4 1.4) (drill 0.7) (layers "*.Cu" "*.Mask") (remove_unused_layers no) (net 11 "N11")))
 (gr_line (start 122.25 53.618227) (end 121.5 52.118227) (stroke (width 0.05) (type default)) (layer "Edge.Cuts"))
 (gr_line (start 123.5 56.618227) (end 122.75 55.118227) (stroke (width 0.05) (type default)) (layer "Edge.Cuts"))
 (gr_line (start 121.5 52.118227) (end 120.5 51.368227) (stroke (width 0.05) (type default)) (layer "Edge.Cuts"))
 (gr_line (start 104.70282 52.25) (end 103.25 52.25) (stroke (width 0.05) (type default)) (layer "Edge.Cuts"))
 (gr_line (start 120.5 51.368227) (end 118.75 51.368227) (stroke (width 0.05) (type default)) (layer "Edge.Cuts"))
 (gr_line (start 122.75 55.118227) (end 122.25 53.618227) (stroke (width 0.05) (type default)) (layer "Edge.Cuts"))
 (gr_line (start 117.25 50.368227) (end 115 50.368227) (stroke (width 0.05) (type default)) (layer "Edge.Cuts"))
 (gr_line (start 121 92.618227) (end 124.75 82.618227) (stroke (width 0.05) (type default)) (layer "Edge.Cuts"))
 (gr_line (start 121.75 68.368227) (end 121.75 66.868227) (stroke (width 0.05) (type default)) (layer "Edge.Cuts"))
 (gr_line (start 96.927145 61.046233) (end 99.259847 61.046233) (stroke (width 0.05) (type default)) (layer "Edge.Cuts"))
 (gr_line (start 96.829948 71.911047) (end 89.200066 90.797179) (stroke (width 0.05) (type default)) (layer "Edge.Cuts"))
 (gr_line (start 115 50.368227) (end 113.75 49.118227) (stroke (width 0.05) (type default)) (layer "Edge.Cuts"))
 (gr_line (start 121.75 66.868227) (end 124.75 59.868227) (stroke (width 0.05) (type default)) (layer "Edge.Cuts"))
 (gr_line (start 77.25 121.618227) (end 92.75 104.618227) (stroke (width 0.05) (type default)) (layer "Edge.Cuts"))
 (gr_line (start 91.241643 113.118227) (end 99.25 104.368227) (stroke (width 0.05) (type default)) (layer "Edge.Cuts"))
 (gr_line (start 102.75 104.368227) (end 109 103.118227) (stroke (width 0.05) (type default)) (layer "Edge.Cuts"))
 (gr_line (start 99.259847 61.046233) (end 96.829948 71.911047) (stroke (width 0.05) (type default)) (layer "Edge.Cuts"))
 (gr_line (start 92.75 104.618227) (end 91.241643 113.118227) (stroke (width 0.05) (type default)) (layer "Edge.Cuts"))
 (gr_line (start 130.75 58.118227) (end 123.5 56.618227) (stroke (width 0.05) (type default)) (layer "Edge.Cuts"))
 (gr_line (start 89.200066 90.797179) (end 85.524897 104.897205) (stroke (width 0.05) (type default)) (layer "Edge.Cuts"))
 (gr_line (start 125 73.868227) (end 121.75 68.368227) (stroke (width 0.05) (type default)) (layer "Edge.Cuts"))
 (gr_line (start 124.75 82.618227) (end 125 73.868227) (stroke (width 0.05) (type default)) (layer "Edge.Cuts"))
 (gr_line (start 85.524897 104.897205) (end 64.25 131.118227) (stroke (width 0.05) (type default)) (layer "Edge.Cuts"))
 (gr_line (start 109 103.118227) (end 116.75 99.118227) (stroke (width 0.05) (type default)) (layer "Edge.Cuts"))
 (gr_line (start 124.75 59.868227) (end 130.75 58.118227) (stroke (width 0.05) (type default)) (layer "Edge.Cuts"))
 (gr_line (start 113.75 49.118227) (end 111.75 49.118227) (stroke (width 0.05) (type default)) (layer "Edge.Cuts"))
 (gr_line (start 99.25 104.368227) (end 102.75 104.368227) (stroke (width 0.05) (type default)) (layer "Edge.Cuts"))
 (gr_line (start 103.25 52.25) (end 96.927145 61.046233) (stroke (width 0.05) (type default)) (layer "Edge.Cuts"))
 (gr_line (start 118.75 51.368227) (end 117.25 50.368227) (stroke (width 0.05) (type default)) (layer "Edge.Cuts"))
 (gr_line (start 116.75 99.118227) (end 121 92.618227) (stroke (width 0.05) (type default)) (layer "Edge.Cuts"))
 (gr_line (start 64.25 131.118227) (end 77.25 121.618227) (stroke (width 0.05) (type default)) (layer "Edge.Cuts"))
 (gr_line (start 111.75 49.118227) (end 104.70282 52.25) (stroke (width 0.05) (type default)) (layer "Edge.Cuts"))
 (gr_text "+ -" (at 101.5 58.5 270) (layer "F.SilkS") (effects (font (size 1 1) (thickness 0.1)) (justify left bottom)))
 (segment (start 101.2839 98.101) (end 95.689 92.5061) (width 0.2) (layer "F.Cu") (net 11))
 (segment (start 105.605628 86.5) (end 104.25 86.5) (width 0.2) (layer "F.Cu") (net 11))
 (segment (start 110.001 90.895372) (end 105.605628 86.5) (width 0.2) (layer "F.Cu") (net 11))
 (segment (start 96.275372 90.499) (end 101.749 90.499) (width 0.2) (layer "F.Cu") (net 11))
 (segment (start 105.5 94.25) (end 107.475628 94.25) (width 0.2) (layer "F.Cu") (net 11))
 (segment (start 104.25 86.5) (end 107.299999 83.450001) (width 0.2) (layer "F.Cu") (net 11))
 (segment (start 118.399 64.149) (end 108.351 64.149) (width 0.2) (layer "F.Cu") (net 11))
 (segment (start 106.149 98.101) (end 101.2839 98.101) (width 0.2) (layer "F.Cu") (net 11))
 (segment (start 101.749 90.499) (end 105.5 94.25) (width 0.2) (layer "F.Cu") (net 11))
 (segment (start 119.5 65.25) (end 118.399 64.149) (width 0.2) (layer "F.Cu") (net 11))
 (segment (start 95.689 91.085372) (end 96.275372 90.499) (width 0.2) (layer "F.Cu") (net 11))
 (segment (start 107.299999 66.799999) (end 106.5 66) (width 0.2) (layer "F.Cu") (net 11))
 (segment (start 113 91.25) (end 106.149 98.101) (width 0.2) (layer "F.Cu") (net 11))
 (segment (start 95.689 92.5061) (end 95.689 91.085372) (width 0.2) (layer "F.Cu") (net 11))
 (segment (start 107.475628 94.25) (end 110.001 91.724628) (width 0.2) (layer "F.Cu") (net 11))
 (segment (start 110.001 91.724628) (end 110.001 90.895372) (width 0.2) (layer "F.Cu") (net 11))
 (segment (start 107.299999 83.450001) (end 107.299999 66.799999) (width 0.2) (layer "F.Cu") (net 11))
 (segment (start 108.351 64.149) (end 106.5 66) (width 0.2) (layer "F.Cu") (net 11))
 (segment (start 118 91.25) (end 118 89) (width 0.2) (layer "F.Cu") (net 7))
 (segment (start 118 89) (end 120.5 86.5) (width 0.2) (layer "F.Cu") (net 7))
 (segment (start 118 91.25) (end 113.351 95.899) (width 0.2) (layer "B.Cu") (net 7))
 (segment (start 105.101 95.899) (end 104 97) (width 0.2) (layer "B.Cu") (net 7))
 (segment (start 113.351 95.899) (end 105.101 95.899) (width 0.2) (layer "B.Cu") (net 7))
 (segment (start 104.75 61.265) (end 108.015 58) (width 0.2) (layer "F.Cu") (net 3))
 (segment (start 108.015 58) (end 114.96 58) (width 0.2) (layer "F.Cu") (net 3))
 (segment (start 93.5 95.62) (end 93.5 89.63) (width 0.2) (layer "F.Cu") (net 5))
 (segment (start 99.204843 72.792413) (end 96.63 75.367256) (width 0.2) (layer "F.Cu") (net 5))
 (segment (start 105.535628 91.31) (end 109 91.31) (width 0.2) (layer "F.Cu") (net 5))
 (segment (start 96.63 75.367256) (end 96.63 86.5) (width 0.2) (layer "F.Cu") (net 5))
 (segment (start 96.63 86.5) (end 100.725628 86.5) (width 0.2) (layer "F.Cu") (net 5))
 (segment (start 93.13 95.99) (end 93.5 95.62) (width 0.2) (layer "F.Cu") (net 5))
 (segment (start 100.725628 86.5) (end 105.535628 91.31) (width 0.2) (layer "F.Cu") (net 5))
 (segment (start 99.204843 64.270157) (end 99.204843 72.792413) (width 0.2) (layer "F.Cu") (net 5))
 (segment (start 93.5 89.63) (end 96.63 86.5) (width 0.2) (layer "F.Cu") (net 5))
 (segment (start 104.75 58.725) (end 99.204843 64.270157) (width 0.2) (layer "F.Cu") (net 5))
 (segment (start 93.13 99.5) (end 93.13 95.99) (width 0.2) (layer "F.Cu") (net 5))
 (segment (start 109 91.31) (end 112.88 87.43) (width 0.2) (layer "B.Cu") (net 5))
 (segment (start 112.88 87.43) (end 112.88 86.5) (width 0.2) (layer "B.Cu") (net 5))
 (segment (start 106.5 99.5) (end 100.75 99.5) (width 0.2) (layer "F.Cu") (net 9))
 (segment (start 109 97) (end 106.5 99.5) (width 0.2) (layer "F.Cu") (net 9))
 (segment (start 103.54395 98.101) (end 102.899 97.45605) (width 0.2) (layer "B.Cu") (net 9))
 (segment (start 102.899 97.45605) (end 102.899 92.911) (width 0.2) (layer "B.Cu") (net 9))
 (segment (start 107.899 98.101) (end 103.54395 98.101) (width 0.2) (layer "B.Cu") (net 9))
 (segment (start 109 97) (end 107.899 98.101) (width 0.2) (layer "B.Cu") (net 9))
 (segment (start 102.899 92.911) (end 104.31 91.5) (width 0.2) (layer "B.Cu") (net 9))
 (segment (start 99.25 95.5) (end 96.69 92.94) (width 0.2) (layer "F.Cu") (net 10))
 (segment (start 115.25 72.25) (end 111 76.5) (width 0.2) (layer "F.Cu") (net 10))
 (segment (start 111 92.25) (end 107.75 95.5) (width 0.2) (layer "F.Cu") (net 10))
 (segment (start 111 76.5) (end 111 92.25) (width 0.2) (layer "F.Cu") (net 10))
 (segment (start 107.75 95.5) (end 99.25 95.5) (width 0.2) (layer "F.Cu") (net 10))
 (segment (start 115.25 66) (end 115.25 72.25) (width 0.2) (layer "F.Cu") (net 10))
 (segment (start 114.5 65.25) (end 115.25 66) (width 0.2) (layer "F.Cu") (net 10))
 (segment (start 96.69 92.94) (end 96.69 91.5) (width 0.2) (layer "F.Cu") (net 10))
 (segment (start 105.94 74.56) (end 104.75 75.75) (width 0.2) (layer "F.Cu") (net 8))
 (segment (start 104.75 75.75) (end 98.25 75.75) (width 0.2) (layer "F.Cu") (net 8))
 (segment (start 105.94 70.44) (end 105.94 71) (width 0.2) (layer "F.Cu") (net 8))
 (segment (start 105.94 71) (end 105.94 74.56) (width 0.2) (layer "F.Cu") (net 8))
 (segment (start 101.5 66) (end 105.94 70.44) (width 0.2) (layer "F.Cu") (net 8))
 (segment (start 98.25 80.25) (end 104.75 80.25) (width 0.2) (layer "F.Cu") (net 6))
 (segment (start 98.25 83.25) (end 98.25 80.25) (width 0.2) (layer "B.Cu") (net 6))
 (segment (start 93.5 88) (end 98.25 83.25) (width 0.2) (layer "B.Cu") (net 6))
 (segment (start 115.25 80.5) (end 121.75 80.5) (width 0.2) (layer "F.Cu") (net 2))
 (segment (start 109 83.69) (end 112.06 83.69) (width 0.2) (layer "B.Cu") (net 2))
 (segment (start 112.06 83.69) (end 115.25 80.5) (width 0.2) (layer "B.Cu") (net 2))
 (segment (start 115.25 76) (end 121.75 76) (width 0.2) (layer "F.Cu") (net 1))
 (segment (start 113.56 74.31) (end 113.56 71) (width 0.2) (layer "B.Cu") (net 1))
 (segment (start 115.25 76) (end 113.56 74.31) (width 0.2) (layer "B.Cu") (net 1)))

